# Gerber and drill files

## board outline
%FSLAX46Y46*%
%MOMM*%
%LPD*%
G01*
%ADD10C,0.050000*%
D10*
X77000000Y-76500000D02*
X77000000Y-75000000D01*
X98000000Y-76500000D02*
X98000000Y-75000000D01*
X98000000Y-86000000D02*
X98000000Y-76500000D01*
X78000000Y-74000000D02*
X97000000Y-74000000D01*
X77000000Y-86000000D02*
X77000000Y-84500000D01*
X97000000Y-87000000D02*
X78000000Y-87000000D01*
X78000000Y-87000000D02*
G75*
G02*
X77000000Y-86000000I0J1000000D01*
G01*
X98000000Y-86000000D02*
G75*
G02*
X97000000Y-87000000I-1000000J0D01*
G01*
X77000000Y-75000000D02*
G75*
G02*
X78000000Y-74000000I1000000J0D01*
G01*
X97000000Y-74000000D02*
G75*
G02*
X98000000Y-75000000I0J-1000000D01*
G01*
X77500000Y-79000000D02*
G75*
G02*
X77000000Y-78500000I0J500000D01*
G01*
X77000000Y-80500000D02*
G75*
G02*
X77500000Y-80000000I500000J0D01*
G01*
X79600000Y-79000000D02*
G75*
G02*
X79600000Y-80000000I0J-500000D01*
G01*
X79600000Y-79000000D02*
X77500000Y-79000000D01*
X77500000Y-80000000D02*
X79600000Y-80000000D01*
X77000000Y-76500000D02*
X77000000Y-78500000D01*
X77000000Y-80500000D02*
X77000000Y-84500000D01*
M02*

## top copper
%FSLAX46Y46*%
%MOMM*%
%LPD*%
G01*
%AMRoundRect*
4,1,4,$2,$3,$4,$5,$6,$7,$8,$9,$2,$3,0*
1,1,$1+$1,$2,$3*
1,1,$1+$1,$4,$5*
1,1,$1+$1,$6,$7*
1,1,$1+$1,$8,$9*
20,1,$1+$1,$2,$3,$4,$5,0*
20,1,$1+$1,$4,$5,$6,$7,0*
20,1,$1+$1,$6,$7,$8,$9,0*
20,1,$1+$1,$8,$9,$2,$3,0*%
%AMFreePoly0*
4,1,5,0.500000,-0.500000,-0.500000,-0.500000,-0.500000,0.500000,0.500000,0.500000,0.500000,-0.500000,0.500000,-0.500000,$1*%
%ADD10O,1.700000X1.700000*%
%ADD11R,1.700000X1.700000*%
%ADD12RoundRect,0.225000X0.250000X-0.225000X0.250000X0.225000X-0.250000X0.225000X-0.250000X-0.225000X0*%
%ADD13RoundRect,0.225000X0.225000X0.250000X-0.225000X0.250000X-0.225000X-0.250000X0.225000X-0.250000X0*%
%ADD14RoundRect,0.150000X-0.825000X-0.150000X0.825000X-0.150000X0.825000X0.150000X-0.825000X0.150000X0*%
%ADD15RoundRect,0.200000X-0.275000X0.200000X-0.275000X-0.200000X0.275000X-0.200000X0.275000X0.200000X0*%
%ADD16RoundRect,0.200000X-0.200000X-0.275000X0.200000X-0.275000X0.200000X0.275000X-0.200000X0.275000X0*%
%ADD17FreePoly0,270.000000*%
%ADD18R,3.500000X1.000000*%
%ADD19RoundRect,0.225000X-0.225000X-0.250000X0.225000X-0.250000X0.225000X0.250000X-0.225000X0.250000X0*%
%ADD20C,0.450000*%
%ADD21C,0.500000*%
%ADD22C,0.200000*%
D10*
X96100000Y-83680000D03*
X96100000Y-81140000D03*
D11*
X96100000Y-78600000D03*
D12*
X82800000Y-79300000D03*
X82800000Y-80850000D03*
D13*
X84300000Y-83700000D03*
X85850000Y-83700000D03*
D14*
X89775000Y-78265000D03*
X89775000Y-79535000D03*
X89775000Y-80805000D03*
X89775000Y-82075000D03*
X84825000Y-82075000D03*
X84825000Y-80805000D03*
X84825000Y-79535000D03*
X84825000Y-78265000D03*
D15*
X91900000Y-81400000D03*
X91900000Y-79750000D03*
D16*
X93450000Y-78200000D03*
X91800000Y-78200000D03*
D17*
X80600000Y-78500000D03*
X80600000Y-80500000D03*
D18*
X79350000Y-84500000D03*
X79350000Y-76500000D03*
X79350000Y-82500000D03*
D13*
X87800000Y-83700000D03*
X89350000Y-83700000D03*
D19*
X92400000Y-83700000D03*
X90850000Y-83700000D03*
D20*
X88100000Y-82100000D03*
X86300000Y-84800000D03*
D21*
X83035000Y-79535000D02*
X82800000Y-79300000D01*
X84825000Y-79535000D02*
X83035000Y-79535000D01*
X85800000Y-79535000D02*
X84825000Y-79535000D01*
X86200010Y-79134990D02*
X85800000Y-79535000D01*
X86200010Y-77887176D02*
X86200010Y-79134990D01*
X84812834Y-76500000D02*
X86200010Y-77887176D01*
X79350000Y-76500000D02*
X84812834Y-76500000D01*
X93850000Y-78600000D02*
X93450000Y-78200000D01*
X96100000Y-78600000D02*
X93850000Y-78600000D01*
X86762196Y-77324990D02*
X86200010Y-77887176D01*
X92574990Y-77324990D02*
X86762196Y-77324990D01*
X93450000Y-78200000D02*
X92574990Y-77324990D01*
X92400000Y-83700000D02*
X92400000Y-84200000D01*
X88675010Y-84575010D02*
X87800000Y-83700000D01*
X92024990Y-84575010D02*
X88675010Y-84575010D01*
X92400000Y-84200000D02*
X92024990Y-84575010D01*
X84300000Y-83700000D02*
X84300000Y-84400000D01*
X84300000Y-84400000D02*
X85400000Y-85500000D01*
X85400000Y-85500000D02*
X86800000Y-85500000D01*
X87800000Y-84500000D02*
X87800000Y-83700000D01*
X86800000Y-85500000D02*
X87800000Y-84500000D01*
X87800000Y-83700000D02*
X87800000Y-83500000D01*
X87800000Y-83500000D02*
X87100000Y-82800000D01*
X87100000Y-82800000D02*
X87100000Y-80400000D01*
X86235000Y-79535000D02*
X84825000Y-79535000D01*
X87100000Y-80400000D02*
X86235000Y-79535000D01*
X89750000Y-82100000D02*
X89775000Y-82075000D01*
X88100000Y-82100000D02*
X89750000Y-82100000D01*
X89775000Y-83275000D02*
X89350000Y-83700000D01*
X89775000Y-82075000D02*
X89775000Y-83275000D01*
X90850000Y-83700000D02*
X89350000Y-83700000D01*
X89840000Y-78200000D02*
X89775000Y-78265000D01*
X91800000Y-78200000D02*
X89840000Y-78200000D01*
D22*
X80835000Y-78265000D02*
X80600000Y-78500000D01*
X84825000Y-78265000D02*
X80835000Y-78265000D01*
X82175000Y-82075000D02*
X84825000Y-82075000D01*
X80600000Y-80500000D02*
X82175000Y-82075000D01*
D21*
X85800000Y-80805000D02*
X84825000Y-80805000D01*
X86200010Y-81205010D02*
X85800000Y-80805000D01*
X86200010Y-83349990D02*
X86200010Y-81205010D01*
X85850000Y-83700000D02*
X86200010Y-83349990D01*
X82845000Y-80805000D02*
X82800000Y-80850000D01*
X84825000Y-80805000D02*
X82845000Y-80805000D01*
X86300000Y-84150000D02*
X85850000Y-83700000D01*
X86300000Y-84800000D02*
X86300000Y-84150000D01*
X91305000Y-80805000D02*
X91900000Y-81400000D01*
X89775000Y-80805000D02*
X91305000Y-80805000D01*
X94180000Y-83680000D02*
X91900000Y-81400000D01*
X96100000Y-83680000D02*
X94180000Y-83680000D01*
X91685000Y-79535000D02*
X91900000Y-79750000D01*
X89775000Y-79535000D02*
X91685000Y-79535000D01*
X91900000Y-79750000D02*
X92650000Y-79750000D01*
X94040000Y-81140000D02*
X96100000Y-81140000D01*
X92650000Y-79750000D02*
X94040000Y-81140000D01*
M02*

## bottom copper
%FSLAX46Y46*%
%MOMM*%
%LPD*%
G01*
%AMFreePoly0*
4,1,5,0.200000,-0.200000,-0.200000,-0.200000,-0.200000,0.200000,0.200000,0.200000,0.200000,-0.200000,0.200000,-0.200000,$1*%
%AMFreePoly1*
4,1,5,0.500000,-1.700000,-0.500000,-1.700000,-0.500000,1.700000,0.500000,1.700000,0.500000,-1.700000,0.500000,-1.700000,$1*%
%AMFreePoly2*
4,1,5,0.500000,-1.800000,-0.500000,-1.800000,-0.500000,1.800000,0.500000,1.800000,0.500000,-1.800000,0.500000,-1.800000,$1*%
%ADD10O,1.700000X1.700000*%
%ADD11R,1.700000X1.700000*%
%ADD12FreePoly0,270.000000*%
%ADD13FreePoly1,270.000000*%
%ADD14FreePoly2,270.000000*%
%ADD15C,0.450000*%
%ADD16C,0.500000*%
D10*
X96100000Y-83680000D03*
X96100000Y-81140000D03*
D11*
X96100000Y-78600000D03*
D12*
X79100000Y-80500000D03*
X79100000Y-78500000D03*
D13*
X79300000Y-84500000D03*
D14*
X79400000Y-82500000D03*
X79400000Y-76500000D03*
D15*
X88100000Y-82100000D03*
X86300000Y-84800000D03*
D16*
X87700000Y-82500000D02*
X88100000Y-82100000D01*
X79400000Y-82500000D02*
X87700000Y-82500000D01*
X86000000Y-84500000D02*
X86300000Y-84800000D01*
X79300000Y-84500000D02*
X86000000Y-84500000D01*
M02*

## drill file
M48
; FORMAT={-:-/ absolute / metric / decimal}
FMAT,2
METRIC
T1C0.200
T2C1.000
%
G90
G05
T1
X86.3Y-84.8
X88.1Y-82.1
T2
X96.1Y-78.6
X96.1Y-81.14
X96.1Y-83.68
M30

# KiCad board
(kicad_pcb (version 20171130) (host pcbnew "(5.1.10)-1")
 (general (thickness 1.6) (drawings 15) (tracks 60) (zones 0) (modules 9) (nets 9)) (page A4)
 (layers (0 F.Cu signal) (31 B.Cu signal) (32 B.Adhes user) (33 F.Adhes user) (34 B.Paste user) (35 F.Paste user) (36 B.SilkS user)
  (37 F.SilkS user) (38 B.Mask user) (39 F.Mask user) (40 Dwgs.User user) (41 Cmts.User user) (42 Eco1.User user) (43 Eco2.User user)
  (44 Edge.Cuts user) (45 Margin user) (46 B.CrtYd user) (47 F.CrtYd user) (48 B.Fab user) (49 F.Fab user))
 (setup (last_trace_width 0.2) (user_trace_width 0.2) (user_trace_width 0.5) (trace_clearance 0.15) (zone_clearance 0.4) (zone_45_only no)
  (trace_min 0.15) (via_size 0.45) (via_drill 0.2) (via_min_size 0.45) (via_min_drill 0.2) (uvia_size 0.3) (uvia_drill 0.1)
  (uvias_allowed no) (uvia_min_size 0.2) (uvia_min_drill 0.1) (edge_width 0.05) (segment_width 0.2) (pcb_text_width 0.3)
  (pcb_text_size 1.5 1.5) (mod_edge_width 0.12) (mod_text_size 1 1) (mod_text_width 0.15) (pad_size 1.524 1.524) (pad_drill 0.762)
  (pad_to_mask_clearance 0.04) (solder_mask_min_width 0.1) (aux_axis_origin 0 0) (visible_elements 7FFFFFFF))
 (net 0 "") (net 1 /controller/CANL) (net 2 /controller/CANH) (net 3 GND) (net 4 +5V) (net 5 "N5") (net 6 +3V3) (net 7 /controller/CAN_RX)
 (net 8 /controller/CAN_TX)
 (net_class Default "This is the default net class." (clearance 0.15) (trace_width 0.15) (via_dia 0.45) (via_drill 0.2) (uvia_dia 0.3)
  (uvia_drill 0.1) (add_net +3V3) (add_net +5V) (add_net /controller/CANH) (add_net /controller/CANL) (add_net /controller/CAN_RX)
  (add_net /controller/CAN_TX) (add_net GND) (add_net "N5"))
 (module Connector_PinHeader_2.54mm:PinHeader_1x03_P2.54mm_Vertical (layer F.Cu) (at 96.1 78.6)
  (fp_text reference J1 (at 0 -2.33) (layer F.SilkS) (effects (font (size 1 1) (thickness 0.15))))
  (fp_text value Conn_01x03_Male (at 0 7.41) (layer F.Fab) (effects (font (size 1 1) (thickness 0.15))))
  (pad 3 thru_hole oval (at 0 5.08) (size 1.7 1.7) (drill 1) (layers *.Cu *.Mask) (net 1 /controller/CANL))
  (pad 2 thru_hole oval (at 0 2.54) (size 1.7 1.7) (drill 1) (layers *.Cu *.Mask) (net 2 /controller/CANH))
  (pad 1 thru_hole rect (at 0 0) (size 1.7 1.7) (drill 1) (layers *.Cu *.Mask) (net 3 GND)))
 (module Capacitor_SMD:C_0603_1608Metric (layer F.Cu) (at 82.8 80.075 90)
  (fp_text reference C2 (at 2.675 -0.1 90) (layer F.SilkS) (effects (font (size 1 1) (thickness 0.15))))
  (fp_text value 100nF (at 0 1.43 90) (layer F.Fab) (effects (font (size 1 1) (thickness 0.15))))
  (pad 2 smd roundrect (at 0.775 0 90) (size 0.9 0.95) (layers F.Cu F.Paste F.Mask) (roundrect_rratio 0.25) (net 3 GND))
  (pad 1 smd roundrect (at -0.775 0 90) (size 0.9 0.95) (layers F.Cu F.Paste F.Mask) (roundrect_rratio 0.25) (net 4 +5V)))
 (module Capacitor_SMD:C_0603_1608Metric (layer F.Cu) (at 85.075 83.7 180)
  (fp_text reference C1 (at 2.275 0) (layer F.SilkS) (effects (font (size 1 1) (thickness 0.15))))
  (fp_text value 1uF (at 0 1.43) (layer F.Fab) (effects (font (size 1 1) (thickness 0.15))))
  (pad 2 smd roundrect (at 0.775 0 180) (size 0.9 0.95) (layers F.Cu F.Paste F.Mask) (roundrect_rratio 0.25) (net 3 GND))
  (pad 1 smd roundrect (at -0.775 0 180) (size 0.9 0.95) (layers F.Cu F.Paste F.Mask) (roundrect_rratio 0.25) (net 4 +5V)))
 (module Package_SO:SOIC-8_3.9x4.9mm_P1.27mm (layer F.Cu) (at 87.3 80.17)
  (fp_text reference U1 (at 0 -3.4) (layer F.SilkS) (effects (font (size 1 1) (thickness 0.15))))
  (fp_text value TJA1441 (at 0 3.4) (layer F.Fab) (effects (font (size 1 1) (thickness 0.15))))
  (pad 8 smd roundrect (at 2.475 -1.905) (size 1.95 0.6) (layers F.Cu F.Paste F.Mask) (roundrect_rratio 0.25) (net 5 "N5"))
  (pad 7 smd roundrect (at 2.475 -0.635) (size 1.95 0.6) (layers F.Cu F.Paste F.Mask) (roundrect_rratio 0.25) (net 2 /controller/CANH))
  (pad 6 smd roundrect (at 2.475 0.635) (size 1.95 0.6) (layers F.Cu F.Paste F.Mask) (roundrect_rratio 0.25) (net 1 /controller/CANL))
  (pad 5 smd roundrect (at 2.475 1.905) (size 1.95 0.6) (layers F.Cu F.Paste F.Mask) (roundrect_rratio 0.25) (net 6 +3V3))
  (pad 4 smd roundrect (at -2.475 1.905) (size 1.95 0.6) (layers F.Cu F.Paste F.Mask) (roundrect_rratio 0.25) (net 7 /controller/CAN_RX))
  (pad 3 smd roundrect (at -2.475 0.635) (size 1.95 0.6) (layers F.Cu F.Paste F.Mask) (roundrect_rratio 0.25) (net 4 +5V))
  (pad 2 smd roundrect (at -2.475 -0.635) (size 1.95 0.6) (layers F.Cu F.Paste F.Mask) (roundrect_rratio 0.25) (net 3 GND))
  (pad 1 smd roundrect (at -2.475 -1.905) (size 1.95 0.6) (layers F.Cu F.Paste F.Mask) (roundrect_rratio 0.25) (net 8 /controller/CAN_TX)))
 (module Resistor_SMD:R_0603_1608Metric (layer F.Cu) (at 91.9 80.575 270)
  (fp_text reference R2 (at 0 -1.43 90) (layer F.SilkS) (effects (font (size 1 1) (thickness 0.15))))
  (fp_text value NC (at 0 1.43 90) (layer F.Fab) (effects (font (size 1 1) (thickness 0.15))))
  (pad 2 smd roundrect (at 0.825 0 270) (size 0.8 0.95) (layers F.Cu F.Paste F.Mask) (roundrect_rratio 0.25) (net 1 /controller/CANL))
  (pad 1 smd roundrect (at -0.825 0 270) (size 0.8 0.95) (layers F.Cu F.Paste F.Mask) (roundrect_rratio 0.25) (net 2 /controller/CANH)))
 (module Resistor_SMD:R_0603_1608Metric (layer F.Cu) (at 92.625 78.2)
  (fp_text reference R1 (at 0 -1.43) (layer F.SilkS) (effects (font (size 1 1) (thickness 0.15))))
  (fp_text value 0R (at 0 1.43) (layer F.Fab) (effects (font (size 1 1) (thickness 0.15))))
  (pad 2 smd roundrect (at 0.825 0) (size 0.8 0.95) (layers F.Cu F.Paste F.Mask) (roundrect_rratio 0.25) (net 3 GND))
  (pad 1 smd roundrect (at -0.825 0) (size 0.8 0.95) (layers F.Cu F.Paste F.Mask) (roundrect_rratio 0.25) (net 5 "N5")))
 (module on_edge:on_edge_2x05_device (layer F.Cu) (at 77 80.5 270)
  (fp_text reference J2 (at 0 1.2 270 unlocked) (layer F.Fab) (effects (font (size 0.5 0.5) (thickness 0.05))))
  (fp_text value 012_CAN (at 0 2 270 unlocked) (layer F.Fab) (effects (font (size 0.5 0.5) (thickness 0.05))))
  (fp_arc (start -2 -0.5) (end -2 0) (angle -90) (layer Edge.Cuts) (width 0.05))
  (fp_arc (start 0 -0.5) (end -0.5 -0.5) (angle -90) (layer Edge.Cuts) (width 0.05))
  (fp_arc (start -1 -2.6) (end -0.5 -2.6) (angle -180) (layer Edge.Cuts) (width 0.05))
  (fp_line (start -1.5 -2.6) (end -1.5 -0.5) (layer Edge.Cuts) (width 0.05))
  (fp_line (start -0.5 -0.5) (end -0.5 -2.6) (layer Edge.Cuts) (width 0.05))
  (fp_line (start -4 0) (end -2 0) (layer Edge.Cuts) (width 0.05))
  (fp_line (start 0 0) (end 4 0) (layer Edge.Cuts) (width 0.05))
  (pad 2 smd custom (at -2 -3.6 270) (size 1 1) (layers F.Cu F.Mask) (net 8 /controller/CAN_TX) (zone_connect 0)
   (options (clearance outline) (anchor rect)) (primitives))
  (pad 3 smd custom (at 0 -3.6 270) (size 1 1) (layers F.Cu F.Mask) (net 7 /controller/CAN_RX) (zone_connect 0)
   (options (clearance outline) (anchor rect)) (primitives))
  (pad 8 smd custom (at 0 -2.1 270) (size 0.4 0.4) (layers B.Cu B.Mask) (zone_connect 0) (options (clearance outline) (anchor rect))
   (primitives))
  (pad 7 smd custom (at -2 -2.1 270) (size 0.4 0.4) (layers B.Cu B.Mask) (zone_connect 0) (options (clearance outline) (anchor rect))
   (primitives))
  (pad 10 smd custom (at 4 -2.3 270) (size 1 3.4) (layers B.Cu B.Mask) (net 4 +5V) (zone_connect 0)
   (options (clearance outline) (anchor rect)) (primitives))
  (pad 9 smd custom (at 2 -2.4 270) (size 1 3.6) (layers B.Cu B.Mask) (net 6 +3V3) (zone_connect 0)
   (options (clearance outline) (anchor rect)) (primitives))
  (pad 6 smd custom (at -4 -2.4 270) (size 1 3.6) (layers B.Cu B.Mask) (zone_connect 0) (options (clearance outline) (anchor rect))
   (primitives))
  (pad 5 smd rect (at 4 -2.35 90) (size 1 3.5) (layers F.Cu F.Mask) (zone_connect 0))
  (pad 1 smd rect (at -4 -2.35 90) (size 1 3.5) (layers F.Cu F.Mask) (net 3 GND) (zone_connect 0))
  (pad 4 smd rect (at 2 -2.35 90) (size 1 3.5) (layers F.Cu F.Mask) (zone_connect 0)))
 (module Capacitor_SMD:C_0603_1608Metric (layer F.Cu) (at 88.575 83.7 180)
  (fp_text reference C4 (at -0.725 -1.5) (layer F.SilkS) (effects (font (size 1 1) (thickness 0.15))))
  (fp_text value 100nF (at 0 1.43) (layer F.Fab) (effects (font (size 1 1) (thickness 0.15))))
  (pad 2 smd roundrect (at 0.775 0 180) (size 0.9 0.95) (layers F.Cu F.Paste F.Mask) (roundrect_rratio 0.25) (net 3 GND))
  (pad 1 smd roundrect (at -0.775 0 180) (size 0.9 0.95) (layers F.Cu F.Paste F.Mask) (roundrect_rratio 0.25) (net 6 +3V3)))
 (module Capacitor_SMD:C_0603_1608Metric (layer F.Cu) (at 91.625 83.7)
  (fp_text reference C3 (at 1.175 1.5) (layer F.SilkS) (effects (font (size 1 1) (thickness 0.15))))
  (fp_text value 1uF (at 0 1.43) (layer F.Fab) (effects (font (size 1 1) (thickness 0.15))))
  (pad 2 smd roundrect (at 0.775 0) (size 0.9 0.95) (layers F.Cu F.Paste F.Mask) (roundrect_rratio 0.25) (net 3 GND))
  (pad 1 smd roundrect (at -0.775 0) (size 0.9 0.95) (layers F.Cu F.Paste F.Mask) (roundrect_rratio 0.25) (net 6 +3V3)))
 (gr_line (start 77 76.5) (end 77 75) (layer Edge.Cuts) (width 0.05))
 (gr_line (start 98 76.5) (end 98 75) (layer Edge.Cuts) (width 0.05))
 (gr_line (start 98 86) (end 98 76.5) (layer Edge.Cuts) (width 0.05))
 (gr_line (start 78 74) (end 97 74) (layer Edge.Cuts) (width 0.05))
 (gr_line (start 77 86) (end 77 84.5) (layer Edge.Cuts) (width 0.05))
 (gr_line (start 97 87) (end 78 87) (layer Edge.Cuts) (width 0.05))
 (gr_arc (start 78 86) (end 77 86) (angle -90) (layer Edge.Cuts) (width 0.05))
 (gr_arc (start 97 86) (end 97 87) (angle -90) (layer Edge.Cuts) (width 0.05))
 (gr_arc (start 78 75) (end 78 74) (angle -90) (layer Edge.Cuts) (width 0.05))
 (gr_arc (start 97 75) (end 98 75) (angle -90) (layer Edge.Cuts) (width 0.05))
 (segment (start 83.035 79.535) (end 82.8 79.3) (width 0.5) (layer F.Cu) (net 3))
 (segment (start 84.825 79.535) (end 83.035 79.535) (width 0.5) (layer F.Cu) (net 3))
 (segment (start 85.8 79.535) (end 84.825 79.535) (width 0.5) (layer F.Cu) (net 3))
 (segment (start 86.20001 79.13499) (end 85.8 79.535) (width 0.5) (layer F.Cu) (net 3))
 (segment (start 86.20001 77.887176) (end 86.20001 79.13499) (width 0.5) (layer F.Cu) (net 3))
 (segment (start 84.812834 76.5) (end 86.20001 77.887176) (width 0.5) (layer F.Cu) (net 3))
 (segment (start 79.35 76.5) (end 84.812834 76.5) (width 0.5) (layer F.Cu) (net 3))
 (segment (start 93.85 78.6) (end 93.45 78.2) (width 0.5) (layer F.Cu) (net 3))
 (segment (start 96.1 78.6) (end 93.85 78.6) (width 0.5) (layer F.Cu) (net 3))
 (segment (start 86.762196 77.32499) (end 86.20001 77.887176) (width 0.5) (layer F.Cu) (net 3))
 (segment (start 92.57499 77.32499) (end 86.762196 77.32499) (width 0.5) (layer F.Cu) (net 3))
 (segment (start 93.45 78.2) (end 92.57499 77.32499) (width 0.5) (layer F.Cu) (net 3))
 (segment (start 92.4 83.7) (end 92.4 84.2) (width 0.5) (layer F.Cu) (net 3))
 (segment (start 88.67501 84.57501) (end 87.8 83.7) (width 0.5) (layer F.Cu) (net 3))
 (segment (start 92.02499 84.57501) (end 88.67501 84.57501) (width 0.5) (layer F.Cu) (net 3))
 (segment (start 92.4 84.2) (end 92.02499 84.57501) (width 0.5) (layer F.Cu) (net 3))
 (segment (start 84.3 83.7) (end 84.3 84.4) (width 0.5) (layer F.Cu) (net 3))
 (segment (start 84.3 84.4) (end 85.4 85.5) (width 0.5) (layer F.Cu) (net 3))
 (segment (start 85.4 85.5) (end 86.8 85.5) (width 0.5) (layer F.Cu) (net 3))
 (segment (start 87.8 84.5) (end 87.8 83.7) (width 0.5) (layer F.Cu) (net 3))
 (segment (start 86.8 85.5) (end 87.8 84.5) (width 0.5) (layer F.Cu) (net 3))
 (segment (start 87.8 83.7) (end 87.8 83.5) (width 0.5) (layer F.Cu) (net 3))
 (segment (start 87.8 83.5) (end 87.1 82.8) (width 0.5) (layer F.Cu) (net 3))
 (segment (start 87.1 82.8) (end 87.1 80.4) (width 0.5) (layer F.Cu) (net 3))
 (segment (start 86.235 79.535) (end 84.825 79.535) (width 0.5) (layer F.Cu) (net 3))
 (segment (start 87.1 80.4) (end 86.235 79.535) (width 0.5) (layer F.Cu) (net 3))
 (via (at 88.1 82.1) (size 0.45) (drill 0.2) (layers F.Cu B.Cu) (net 6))
 (segment (start 87.7 82.5) (end 88.1 82.1) (width 0.5) (layer B.Cu) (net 6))
 (segment (start 79.4 82.5) (end 87.7 82.5) (width 0.5) (layer B.Cu) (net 6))
 (segment (start 89.75 82.1) (end 89.775 82.075) (width 0.5) (layer F.Cu) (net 6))
 (segment (start 88.1 82.1) (end 89.75 82.1) (width 0.5) (layer F.Cu) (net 6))
 (segment (start 89.775 83.275) (end 89.35 83.7) (width 0.5) (layer F.Cu) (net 6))
 (segment (start 89.775 82.075) (end 89.775 83.275) (width 0.5) (layer F.Cu) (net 6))
 (segment (start 90.85 83.7) (end 89.35 83.7) (width 0.5) (layer F.Cu) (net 6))
 (segment (start 89.84 78.2) (end 89.775 78.265) (width 0.5) (layer F.Cu) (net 5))
 (segment (start 91.8 78.2) (end 89.84 78.2) (width 0.5) (layer F.Cu) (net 5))
 (segment (start 80.835 78.265) (end 80.6 78.5) (width 0.2) (layer F.Cu) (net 8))
 (segment (start 84.825 78.265) (end 80.835 78.265) (width 0.2) (layer F.Cu) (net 8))
 (segment (start 82.175 82.075) (end 84.825 82.075) (width 0.2) (layer F.Cu) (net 7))
 (segment (start 80.6 80.5) (end 82.175 82.075) (width 0.2) (layer F.Cu) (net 7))
 (segment (start 85.8 80.805) (end 84.825 80.805) (width 0.5) (layer F.Cu) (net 4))
 (segment (start 86.20001 81.20501) (end 85.8 80.805) (width 0.5) (layer F.Cu) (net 4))
 (segment (start 86.20001 83.34999) (end 86.20001 81.20501) (width 0.5) (layer F.Cu) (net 4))
 (segment (start 85.85 83.7) (end 86.20001 83.34999) (width 0.5) (layer F.Cu) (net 4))
 (segment (start 82.845 80.805) (end 82.8 80.85) (width 0.5) (layer F.Cu) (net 4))
 (segment (start 84.825 80.805) (end 82.845 80.805) (width 0.5) (layer F.Cu) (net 4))
 (via (at 86.3 84.8) (size 0.45) (drill 0.2) (layers F.Cu B.Cu) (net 4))
 (segment (start 86 84.5) (end 86.3 84.8) (width 0.5) (layer B.Cu) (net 4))
 (segment (start 79.3 84.5) (end 86 84.5) (width 0.5) (layer B.Cu) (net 4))
 (segment (start 86.3 84.15) (end 85.85 83.7) (width 0.5) (layer F.Cu) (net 4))
 (segment (start 86.3 84.8) (end 86.3 84.15) (width 0.5) (layer F.Cu) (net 4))
 (segment (start 91.305 80.805) (end 91.9 81.4) (width 0.5) (layer F.Cu) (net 1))
 (segment (start 89.775 80.805) (end 91.305 80.805) (width 0.5) (layer F.Cu) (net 1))
 (segment (start 94.18 83.68) (end 91.9 81.4) (width 0.5) (layer F.Cu) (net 1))
 (segment (start 96.1 83.68) (end 94.18 83.68) (width 0.5) (layer F.Cu) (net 1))
 (segment (start 91.685 79.535) (end 91.9 79.75) (width 0.5) (layer F.Cu) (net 2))
 (segment (start 89.775 79.535) (end 91.685 79.535) (width 0.5) (layer F.Cu) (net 2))
 (segment (start 91.9 79.75) (end 92.65 79.75) (width 0.5) (layer F.Cu) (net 2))
 (segment (start 94.04 81.14) (end 96.1 81.14) (width 0.5) (layer F.Cu) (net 2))
 (segment (start 92.65 79.75) (end 94.04 81.14) (width 0.5) (layer F.Cu) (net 2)))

